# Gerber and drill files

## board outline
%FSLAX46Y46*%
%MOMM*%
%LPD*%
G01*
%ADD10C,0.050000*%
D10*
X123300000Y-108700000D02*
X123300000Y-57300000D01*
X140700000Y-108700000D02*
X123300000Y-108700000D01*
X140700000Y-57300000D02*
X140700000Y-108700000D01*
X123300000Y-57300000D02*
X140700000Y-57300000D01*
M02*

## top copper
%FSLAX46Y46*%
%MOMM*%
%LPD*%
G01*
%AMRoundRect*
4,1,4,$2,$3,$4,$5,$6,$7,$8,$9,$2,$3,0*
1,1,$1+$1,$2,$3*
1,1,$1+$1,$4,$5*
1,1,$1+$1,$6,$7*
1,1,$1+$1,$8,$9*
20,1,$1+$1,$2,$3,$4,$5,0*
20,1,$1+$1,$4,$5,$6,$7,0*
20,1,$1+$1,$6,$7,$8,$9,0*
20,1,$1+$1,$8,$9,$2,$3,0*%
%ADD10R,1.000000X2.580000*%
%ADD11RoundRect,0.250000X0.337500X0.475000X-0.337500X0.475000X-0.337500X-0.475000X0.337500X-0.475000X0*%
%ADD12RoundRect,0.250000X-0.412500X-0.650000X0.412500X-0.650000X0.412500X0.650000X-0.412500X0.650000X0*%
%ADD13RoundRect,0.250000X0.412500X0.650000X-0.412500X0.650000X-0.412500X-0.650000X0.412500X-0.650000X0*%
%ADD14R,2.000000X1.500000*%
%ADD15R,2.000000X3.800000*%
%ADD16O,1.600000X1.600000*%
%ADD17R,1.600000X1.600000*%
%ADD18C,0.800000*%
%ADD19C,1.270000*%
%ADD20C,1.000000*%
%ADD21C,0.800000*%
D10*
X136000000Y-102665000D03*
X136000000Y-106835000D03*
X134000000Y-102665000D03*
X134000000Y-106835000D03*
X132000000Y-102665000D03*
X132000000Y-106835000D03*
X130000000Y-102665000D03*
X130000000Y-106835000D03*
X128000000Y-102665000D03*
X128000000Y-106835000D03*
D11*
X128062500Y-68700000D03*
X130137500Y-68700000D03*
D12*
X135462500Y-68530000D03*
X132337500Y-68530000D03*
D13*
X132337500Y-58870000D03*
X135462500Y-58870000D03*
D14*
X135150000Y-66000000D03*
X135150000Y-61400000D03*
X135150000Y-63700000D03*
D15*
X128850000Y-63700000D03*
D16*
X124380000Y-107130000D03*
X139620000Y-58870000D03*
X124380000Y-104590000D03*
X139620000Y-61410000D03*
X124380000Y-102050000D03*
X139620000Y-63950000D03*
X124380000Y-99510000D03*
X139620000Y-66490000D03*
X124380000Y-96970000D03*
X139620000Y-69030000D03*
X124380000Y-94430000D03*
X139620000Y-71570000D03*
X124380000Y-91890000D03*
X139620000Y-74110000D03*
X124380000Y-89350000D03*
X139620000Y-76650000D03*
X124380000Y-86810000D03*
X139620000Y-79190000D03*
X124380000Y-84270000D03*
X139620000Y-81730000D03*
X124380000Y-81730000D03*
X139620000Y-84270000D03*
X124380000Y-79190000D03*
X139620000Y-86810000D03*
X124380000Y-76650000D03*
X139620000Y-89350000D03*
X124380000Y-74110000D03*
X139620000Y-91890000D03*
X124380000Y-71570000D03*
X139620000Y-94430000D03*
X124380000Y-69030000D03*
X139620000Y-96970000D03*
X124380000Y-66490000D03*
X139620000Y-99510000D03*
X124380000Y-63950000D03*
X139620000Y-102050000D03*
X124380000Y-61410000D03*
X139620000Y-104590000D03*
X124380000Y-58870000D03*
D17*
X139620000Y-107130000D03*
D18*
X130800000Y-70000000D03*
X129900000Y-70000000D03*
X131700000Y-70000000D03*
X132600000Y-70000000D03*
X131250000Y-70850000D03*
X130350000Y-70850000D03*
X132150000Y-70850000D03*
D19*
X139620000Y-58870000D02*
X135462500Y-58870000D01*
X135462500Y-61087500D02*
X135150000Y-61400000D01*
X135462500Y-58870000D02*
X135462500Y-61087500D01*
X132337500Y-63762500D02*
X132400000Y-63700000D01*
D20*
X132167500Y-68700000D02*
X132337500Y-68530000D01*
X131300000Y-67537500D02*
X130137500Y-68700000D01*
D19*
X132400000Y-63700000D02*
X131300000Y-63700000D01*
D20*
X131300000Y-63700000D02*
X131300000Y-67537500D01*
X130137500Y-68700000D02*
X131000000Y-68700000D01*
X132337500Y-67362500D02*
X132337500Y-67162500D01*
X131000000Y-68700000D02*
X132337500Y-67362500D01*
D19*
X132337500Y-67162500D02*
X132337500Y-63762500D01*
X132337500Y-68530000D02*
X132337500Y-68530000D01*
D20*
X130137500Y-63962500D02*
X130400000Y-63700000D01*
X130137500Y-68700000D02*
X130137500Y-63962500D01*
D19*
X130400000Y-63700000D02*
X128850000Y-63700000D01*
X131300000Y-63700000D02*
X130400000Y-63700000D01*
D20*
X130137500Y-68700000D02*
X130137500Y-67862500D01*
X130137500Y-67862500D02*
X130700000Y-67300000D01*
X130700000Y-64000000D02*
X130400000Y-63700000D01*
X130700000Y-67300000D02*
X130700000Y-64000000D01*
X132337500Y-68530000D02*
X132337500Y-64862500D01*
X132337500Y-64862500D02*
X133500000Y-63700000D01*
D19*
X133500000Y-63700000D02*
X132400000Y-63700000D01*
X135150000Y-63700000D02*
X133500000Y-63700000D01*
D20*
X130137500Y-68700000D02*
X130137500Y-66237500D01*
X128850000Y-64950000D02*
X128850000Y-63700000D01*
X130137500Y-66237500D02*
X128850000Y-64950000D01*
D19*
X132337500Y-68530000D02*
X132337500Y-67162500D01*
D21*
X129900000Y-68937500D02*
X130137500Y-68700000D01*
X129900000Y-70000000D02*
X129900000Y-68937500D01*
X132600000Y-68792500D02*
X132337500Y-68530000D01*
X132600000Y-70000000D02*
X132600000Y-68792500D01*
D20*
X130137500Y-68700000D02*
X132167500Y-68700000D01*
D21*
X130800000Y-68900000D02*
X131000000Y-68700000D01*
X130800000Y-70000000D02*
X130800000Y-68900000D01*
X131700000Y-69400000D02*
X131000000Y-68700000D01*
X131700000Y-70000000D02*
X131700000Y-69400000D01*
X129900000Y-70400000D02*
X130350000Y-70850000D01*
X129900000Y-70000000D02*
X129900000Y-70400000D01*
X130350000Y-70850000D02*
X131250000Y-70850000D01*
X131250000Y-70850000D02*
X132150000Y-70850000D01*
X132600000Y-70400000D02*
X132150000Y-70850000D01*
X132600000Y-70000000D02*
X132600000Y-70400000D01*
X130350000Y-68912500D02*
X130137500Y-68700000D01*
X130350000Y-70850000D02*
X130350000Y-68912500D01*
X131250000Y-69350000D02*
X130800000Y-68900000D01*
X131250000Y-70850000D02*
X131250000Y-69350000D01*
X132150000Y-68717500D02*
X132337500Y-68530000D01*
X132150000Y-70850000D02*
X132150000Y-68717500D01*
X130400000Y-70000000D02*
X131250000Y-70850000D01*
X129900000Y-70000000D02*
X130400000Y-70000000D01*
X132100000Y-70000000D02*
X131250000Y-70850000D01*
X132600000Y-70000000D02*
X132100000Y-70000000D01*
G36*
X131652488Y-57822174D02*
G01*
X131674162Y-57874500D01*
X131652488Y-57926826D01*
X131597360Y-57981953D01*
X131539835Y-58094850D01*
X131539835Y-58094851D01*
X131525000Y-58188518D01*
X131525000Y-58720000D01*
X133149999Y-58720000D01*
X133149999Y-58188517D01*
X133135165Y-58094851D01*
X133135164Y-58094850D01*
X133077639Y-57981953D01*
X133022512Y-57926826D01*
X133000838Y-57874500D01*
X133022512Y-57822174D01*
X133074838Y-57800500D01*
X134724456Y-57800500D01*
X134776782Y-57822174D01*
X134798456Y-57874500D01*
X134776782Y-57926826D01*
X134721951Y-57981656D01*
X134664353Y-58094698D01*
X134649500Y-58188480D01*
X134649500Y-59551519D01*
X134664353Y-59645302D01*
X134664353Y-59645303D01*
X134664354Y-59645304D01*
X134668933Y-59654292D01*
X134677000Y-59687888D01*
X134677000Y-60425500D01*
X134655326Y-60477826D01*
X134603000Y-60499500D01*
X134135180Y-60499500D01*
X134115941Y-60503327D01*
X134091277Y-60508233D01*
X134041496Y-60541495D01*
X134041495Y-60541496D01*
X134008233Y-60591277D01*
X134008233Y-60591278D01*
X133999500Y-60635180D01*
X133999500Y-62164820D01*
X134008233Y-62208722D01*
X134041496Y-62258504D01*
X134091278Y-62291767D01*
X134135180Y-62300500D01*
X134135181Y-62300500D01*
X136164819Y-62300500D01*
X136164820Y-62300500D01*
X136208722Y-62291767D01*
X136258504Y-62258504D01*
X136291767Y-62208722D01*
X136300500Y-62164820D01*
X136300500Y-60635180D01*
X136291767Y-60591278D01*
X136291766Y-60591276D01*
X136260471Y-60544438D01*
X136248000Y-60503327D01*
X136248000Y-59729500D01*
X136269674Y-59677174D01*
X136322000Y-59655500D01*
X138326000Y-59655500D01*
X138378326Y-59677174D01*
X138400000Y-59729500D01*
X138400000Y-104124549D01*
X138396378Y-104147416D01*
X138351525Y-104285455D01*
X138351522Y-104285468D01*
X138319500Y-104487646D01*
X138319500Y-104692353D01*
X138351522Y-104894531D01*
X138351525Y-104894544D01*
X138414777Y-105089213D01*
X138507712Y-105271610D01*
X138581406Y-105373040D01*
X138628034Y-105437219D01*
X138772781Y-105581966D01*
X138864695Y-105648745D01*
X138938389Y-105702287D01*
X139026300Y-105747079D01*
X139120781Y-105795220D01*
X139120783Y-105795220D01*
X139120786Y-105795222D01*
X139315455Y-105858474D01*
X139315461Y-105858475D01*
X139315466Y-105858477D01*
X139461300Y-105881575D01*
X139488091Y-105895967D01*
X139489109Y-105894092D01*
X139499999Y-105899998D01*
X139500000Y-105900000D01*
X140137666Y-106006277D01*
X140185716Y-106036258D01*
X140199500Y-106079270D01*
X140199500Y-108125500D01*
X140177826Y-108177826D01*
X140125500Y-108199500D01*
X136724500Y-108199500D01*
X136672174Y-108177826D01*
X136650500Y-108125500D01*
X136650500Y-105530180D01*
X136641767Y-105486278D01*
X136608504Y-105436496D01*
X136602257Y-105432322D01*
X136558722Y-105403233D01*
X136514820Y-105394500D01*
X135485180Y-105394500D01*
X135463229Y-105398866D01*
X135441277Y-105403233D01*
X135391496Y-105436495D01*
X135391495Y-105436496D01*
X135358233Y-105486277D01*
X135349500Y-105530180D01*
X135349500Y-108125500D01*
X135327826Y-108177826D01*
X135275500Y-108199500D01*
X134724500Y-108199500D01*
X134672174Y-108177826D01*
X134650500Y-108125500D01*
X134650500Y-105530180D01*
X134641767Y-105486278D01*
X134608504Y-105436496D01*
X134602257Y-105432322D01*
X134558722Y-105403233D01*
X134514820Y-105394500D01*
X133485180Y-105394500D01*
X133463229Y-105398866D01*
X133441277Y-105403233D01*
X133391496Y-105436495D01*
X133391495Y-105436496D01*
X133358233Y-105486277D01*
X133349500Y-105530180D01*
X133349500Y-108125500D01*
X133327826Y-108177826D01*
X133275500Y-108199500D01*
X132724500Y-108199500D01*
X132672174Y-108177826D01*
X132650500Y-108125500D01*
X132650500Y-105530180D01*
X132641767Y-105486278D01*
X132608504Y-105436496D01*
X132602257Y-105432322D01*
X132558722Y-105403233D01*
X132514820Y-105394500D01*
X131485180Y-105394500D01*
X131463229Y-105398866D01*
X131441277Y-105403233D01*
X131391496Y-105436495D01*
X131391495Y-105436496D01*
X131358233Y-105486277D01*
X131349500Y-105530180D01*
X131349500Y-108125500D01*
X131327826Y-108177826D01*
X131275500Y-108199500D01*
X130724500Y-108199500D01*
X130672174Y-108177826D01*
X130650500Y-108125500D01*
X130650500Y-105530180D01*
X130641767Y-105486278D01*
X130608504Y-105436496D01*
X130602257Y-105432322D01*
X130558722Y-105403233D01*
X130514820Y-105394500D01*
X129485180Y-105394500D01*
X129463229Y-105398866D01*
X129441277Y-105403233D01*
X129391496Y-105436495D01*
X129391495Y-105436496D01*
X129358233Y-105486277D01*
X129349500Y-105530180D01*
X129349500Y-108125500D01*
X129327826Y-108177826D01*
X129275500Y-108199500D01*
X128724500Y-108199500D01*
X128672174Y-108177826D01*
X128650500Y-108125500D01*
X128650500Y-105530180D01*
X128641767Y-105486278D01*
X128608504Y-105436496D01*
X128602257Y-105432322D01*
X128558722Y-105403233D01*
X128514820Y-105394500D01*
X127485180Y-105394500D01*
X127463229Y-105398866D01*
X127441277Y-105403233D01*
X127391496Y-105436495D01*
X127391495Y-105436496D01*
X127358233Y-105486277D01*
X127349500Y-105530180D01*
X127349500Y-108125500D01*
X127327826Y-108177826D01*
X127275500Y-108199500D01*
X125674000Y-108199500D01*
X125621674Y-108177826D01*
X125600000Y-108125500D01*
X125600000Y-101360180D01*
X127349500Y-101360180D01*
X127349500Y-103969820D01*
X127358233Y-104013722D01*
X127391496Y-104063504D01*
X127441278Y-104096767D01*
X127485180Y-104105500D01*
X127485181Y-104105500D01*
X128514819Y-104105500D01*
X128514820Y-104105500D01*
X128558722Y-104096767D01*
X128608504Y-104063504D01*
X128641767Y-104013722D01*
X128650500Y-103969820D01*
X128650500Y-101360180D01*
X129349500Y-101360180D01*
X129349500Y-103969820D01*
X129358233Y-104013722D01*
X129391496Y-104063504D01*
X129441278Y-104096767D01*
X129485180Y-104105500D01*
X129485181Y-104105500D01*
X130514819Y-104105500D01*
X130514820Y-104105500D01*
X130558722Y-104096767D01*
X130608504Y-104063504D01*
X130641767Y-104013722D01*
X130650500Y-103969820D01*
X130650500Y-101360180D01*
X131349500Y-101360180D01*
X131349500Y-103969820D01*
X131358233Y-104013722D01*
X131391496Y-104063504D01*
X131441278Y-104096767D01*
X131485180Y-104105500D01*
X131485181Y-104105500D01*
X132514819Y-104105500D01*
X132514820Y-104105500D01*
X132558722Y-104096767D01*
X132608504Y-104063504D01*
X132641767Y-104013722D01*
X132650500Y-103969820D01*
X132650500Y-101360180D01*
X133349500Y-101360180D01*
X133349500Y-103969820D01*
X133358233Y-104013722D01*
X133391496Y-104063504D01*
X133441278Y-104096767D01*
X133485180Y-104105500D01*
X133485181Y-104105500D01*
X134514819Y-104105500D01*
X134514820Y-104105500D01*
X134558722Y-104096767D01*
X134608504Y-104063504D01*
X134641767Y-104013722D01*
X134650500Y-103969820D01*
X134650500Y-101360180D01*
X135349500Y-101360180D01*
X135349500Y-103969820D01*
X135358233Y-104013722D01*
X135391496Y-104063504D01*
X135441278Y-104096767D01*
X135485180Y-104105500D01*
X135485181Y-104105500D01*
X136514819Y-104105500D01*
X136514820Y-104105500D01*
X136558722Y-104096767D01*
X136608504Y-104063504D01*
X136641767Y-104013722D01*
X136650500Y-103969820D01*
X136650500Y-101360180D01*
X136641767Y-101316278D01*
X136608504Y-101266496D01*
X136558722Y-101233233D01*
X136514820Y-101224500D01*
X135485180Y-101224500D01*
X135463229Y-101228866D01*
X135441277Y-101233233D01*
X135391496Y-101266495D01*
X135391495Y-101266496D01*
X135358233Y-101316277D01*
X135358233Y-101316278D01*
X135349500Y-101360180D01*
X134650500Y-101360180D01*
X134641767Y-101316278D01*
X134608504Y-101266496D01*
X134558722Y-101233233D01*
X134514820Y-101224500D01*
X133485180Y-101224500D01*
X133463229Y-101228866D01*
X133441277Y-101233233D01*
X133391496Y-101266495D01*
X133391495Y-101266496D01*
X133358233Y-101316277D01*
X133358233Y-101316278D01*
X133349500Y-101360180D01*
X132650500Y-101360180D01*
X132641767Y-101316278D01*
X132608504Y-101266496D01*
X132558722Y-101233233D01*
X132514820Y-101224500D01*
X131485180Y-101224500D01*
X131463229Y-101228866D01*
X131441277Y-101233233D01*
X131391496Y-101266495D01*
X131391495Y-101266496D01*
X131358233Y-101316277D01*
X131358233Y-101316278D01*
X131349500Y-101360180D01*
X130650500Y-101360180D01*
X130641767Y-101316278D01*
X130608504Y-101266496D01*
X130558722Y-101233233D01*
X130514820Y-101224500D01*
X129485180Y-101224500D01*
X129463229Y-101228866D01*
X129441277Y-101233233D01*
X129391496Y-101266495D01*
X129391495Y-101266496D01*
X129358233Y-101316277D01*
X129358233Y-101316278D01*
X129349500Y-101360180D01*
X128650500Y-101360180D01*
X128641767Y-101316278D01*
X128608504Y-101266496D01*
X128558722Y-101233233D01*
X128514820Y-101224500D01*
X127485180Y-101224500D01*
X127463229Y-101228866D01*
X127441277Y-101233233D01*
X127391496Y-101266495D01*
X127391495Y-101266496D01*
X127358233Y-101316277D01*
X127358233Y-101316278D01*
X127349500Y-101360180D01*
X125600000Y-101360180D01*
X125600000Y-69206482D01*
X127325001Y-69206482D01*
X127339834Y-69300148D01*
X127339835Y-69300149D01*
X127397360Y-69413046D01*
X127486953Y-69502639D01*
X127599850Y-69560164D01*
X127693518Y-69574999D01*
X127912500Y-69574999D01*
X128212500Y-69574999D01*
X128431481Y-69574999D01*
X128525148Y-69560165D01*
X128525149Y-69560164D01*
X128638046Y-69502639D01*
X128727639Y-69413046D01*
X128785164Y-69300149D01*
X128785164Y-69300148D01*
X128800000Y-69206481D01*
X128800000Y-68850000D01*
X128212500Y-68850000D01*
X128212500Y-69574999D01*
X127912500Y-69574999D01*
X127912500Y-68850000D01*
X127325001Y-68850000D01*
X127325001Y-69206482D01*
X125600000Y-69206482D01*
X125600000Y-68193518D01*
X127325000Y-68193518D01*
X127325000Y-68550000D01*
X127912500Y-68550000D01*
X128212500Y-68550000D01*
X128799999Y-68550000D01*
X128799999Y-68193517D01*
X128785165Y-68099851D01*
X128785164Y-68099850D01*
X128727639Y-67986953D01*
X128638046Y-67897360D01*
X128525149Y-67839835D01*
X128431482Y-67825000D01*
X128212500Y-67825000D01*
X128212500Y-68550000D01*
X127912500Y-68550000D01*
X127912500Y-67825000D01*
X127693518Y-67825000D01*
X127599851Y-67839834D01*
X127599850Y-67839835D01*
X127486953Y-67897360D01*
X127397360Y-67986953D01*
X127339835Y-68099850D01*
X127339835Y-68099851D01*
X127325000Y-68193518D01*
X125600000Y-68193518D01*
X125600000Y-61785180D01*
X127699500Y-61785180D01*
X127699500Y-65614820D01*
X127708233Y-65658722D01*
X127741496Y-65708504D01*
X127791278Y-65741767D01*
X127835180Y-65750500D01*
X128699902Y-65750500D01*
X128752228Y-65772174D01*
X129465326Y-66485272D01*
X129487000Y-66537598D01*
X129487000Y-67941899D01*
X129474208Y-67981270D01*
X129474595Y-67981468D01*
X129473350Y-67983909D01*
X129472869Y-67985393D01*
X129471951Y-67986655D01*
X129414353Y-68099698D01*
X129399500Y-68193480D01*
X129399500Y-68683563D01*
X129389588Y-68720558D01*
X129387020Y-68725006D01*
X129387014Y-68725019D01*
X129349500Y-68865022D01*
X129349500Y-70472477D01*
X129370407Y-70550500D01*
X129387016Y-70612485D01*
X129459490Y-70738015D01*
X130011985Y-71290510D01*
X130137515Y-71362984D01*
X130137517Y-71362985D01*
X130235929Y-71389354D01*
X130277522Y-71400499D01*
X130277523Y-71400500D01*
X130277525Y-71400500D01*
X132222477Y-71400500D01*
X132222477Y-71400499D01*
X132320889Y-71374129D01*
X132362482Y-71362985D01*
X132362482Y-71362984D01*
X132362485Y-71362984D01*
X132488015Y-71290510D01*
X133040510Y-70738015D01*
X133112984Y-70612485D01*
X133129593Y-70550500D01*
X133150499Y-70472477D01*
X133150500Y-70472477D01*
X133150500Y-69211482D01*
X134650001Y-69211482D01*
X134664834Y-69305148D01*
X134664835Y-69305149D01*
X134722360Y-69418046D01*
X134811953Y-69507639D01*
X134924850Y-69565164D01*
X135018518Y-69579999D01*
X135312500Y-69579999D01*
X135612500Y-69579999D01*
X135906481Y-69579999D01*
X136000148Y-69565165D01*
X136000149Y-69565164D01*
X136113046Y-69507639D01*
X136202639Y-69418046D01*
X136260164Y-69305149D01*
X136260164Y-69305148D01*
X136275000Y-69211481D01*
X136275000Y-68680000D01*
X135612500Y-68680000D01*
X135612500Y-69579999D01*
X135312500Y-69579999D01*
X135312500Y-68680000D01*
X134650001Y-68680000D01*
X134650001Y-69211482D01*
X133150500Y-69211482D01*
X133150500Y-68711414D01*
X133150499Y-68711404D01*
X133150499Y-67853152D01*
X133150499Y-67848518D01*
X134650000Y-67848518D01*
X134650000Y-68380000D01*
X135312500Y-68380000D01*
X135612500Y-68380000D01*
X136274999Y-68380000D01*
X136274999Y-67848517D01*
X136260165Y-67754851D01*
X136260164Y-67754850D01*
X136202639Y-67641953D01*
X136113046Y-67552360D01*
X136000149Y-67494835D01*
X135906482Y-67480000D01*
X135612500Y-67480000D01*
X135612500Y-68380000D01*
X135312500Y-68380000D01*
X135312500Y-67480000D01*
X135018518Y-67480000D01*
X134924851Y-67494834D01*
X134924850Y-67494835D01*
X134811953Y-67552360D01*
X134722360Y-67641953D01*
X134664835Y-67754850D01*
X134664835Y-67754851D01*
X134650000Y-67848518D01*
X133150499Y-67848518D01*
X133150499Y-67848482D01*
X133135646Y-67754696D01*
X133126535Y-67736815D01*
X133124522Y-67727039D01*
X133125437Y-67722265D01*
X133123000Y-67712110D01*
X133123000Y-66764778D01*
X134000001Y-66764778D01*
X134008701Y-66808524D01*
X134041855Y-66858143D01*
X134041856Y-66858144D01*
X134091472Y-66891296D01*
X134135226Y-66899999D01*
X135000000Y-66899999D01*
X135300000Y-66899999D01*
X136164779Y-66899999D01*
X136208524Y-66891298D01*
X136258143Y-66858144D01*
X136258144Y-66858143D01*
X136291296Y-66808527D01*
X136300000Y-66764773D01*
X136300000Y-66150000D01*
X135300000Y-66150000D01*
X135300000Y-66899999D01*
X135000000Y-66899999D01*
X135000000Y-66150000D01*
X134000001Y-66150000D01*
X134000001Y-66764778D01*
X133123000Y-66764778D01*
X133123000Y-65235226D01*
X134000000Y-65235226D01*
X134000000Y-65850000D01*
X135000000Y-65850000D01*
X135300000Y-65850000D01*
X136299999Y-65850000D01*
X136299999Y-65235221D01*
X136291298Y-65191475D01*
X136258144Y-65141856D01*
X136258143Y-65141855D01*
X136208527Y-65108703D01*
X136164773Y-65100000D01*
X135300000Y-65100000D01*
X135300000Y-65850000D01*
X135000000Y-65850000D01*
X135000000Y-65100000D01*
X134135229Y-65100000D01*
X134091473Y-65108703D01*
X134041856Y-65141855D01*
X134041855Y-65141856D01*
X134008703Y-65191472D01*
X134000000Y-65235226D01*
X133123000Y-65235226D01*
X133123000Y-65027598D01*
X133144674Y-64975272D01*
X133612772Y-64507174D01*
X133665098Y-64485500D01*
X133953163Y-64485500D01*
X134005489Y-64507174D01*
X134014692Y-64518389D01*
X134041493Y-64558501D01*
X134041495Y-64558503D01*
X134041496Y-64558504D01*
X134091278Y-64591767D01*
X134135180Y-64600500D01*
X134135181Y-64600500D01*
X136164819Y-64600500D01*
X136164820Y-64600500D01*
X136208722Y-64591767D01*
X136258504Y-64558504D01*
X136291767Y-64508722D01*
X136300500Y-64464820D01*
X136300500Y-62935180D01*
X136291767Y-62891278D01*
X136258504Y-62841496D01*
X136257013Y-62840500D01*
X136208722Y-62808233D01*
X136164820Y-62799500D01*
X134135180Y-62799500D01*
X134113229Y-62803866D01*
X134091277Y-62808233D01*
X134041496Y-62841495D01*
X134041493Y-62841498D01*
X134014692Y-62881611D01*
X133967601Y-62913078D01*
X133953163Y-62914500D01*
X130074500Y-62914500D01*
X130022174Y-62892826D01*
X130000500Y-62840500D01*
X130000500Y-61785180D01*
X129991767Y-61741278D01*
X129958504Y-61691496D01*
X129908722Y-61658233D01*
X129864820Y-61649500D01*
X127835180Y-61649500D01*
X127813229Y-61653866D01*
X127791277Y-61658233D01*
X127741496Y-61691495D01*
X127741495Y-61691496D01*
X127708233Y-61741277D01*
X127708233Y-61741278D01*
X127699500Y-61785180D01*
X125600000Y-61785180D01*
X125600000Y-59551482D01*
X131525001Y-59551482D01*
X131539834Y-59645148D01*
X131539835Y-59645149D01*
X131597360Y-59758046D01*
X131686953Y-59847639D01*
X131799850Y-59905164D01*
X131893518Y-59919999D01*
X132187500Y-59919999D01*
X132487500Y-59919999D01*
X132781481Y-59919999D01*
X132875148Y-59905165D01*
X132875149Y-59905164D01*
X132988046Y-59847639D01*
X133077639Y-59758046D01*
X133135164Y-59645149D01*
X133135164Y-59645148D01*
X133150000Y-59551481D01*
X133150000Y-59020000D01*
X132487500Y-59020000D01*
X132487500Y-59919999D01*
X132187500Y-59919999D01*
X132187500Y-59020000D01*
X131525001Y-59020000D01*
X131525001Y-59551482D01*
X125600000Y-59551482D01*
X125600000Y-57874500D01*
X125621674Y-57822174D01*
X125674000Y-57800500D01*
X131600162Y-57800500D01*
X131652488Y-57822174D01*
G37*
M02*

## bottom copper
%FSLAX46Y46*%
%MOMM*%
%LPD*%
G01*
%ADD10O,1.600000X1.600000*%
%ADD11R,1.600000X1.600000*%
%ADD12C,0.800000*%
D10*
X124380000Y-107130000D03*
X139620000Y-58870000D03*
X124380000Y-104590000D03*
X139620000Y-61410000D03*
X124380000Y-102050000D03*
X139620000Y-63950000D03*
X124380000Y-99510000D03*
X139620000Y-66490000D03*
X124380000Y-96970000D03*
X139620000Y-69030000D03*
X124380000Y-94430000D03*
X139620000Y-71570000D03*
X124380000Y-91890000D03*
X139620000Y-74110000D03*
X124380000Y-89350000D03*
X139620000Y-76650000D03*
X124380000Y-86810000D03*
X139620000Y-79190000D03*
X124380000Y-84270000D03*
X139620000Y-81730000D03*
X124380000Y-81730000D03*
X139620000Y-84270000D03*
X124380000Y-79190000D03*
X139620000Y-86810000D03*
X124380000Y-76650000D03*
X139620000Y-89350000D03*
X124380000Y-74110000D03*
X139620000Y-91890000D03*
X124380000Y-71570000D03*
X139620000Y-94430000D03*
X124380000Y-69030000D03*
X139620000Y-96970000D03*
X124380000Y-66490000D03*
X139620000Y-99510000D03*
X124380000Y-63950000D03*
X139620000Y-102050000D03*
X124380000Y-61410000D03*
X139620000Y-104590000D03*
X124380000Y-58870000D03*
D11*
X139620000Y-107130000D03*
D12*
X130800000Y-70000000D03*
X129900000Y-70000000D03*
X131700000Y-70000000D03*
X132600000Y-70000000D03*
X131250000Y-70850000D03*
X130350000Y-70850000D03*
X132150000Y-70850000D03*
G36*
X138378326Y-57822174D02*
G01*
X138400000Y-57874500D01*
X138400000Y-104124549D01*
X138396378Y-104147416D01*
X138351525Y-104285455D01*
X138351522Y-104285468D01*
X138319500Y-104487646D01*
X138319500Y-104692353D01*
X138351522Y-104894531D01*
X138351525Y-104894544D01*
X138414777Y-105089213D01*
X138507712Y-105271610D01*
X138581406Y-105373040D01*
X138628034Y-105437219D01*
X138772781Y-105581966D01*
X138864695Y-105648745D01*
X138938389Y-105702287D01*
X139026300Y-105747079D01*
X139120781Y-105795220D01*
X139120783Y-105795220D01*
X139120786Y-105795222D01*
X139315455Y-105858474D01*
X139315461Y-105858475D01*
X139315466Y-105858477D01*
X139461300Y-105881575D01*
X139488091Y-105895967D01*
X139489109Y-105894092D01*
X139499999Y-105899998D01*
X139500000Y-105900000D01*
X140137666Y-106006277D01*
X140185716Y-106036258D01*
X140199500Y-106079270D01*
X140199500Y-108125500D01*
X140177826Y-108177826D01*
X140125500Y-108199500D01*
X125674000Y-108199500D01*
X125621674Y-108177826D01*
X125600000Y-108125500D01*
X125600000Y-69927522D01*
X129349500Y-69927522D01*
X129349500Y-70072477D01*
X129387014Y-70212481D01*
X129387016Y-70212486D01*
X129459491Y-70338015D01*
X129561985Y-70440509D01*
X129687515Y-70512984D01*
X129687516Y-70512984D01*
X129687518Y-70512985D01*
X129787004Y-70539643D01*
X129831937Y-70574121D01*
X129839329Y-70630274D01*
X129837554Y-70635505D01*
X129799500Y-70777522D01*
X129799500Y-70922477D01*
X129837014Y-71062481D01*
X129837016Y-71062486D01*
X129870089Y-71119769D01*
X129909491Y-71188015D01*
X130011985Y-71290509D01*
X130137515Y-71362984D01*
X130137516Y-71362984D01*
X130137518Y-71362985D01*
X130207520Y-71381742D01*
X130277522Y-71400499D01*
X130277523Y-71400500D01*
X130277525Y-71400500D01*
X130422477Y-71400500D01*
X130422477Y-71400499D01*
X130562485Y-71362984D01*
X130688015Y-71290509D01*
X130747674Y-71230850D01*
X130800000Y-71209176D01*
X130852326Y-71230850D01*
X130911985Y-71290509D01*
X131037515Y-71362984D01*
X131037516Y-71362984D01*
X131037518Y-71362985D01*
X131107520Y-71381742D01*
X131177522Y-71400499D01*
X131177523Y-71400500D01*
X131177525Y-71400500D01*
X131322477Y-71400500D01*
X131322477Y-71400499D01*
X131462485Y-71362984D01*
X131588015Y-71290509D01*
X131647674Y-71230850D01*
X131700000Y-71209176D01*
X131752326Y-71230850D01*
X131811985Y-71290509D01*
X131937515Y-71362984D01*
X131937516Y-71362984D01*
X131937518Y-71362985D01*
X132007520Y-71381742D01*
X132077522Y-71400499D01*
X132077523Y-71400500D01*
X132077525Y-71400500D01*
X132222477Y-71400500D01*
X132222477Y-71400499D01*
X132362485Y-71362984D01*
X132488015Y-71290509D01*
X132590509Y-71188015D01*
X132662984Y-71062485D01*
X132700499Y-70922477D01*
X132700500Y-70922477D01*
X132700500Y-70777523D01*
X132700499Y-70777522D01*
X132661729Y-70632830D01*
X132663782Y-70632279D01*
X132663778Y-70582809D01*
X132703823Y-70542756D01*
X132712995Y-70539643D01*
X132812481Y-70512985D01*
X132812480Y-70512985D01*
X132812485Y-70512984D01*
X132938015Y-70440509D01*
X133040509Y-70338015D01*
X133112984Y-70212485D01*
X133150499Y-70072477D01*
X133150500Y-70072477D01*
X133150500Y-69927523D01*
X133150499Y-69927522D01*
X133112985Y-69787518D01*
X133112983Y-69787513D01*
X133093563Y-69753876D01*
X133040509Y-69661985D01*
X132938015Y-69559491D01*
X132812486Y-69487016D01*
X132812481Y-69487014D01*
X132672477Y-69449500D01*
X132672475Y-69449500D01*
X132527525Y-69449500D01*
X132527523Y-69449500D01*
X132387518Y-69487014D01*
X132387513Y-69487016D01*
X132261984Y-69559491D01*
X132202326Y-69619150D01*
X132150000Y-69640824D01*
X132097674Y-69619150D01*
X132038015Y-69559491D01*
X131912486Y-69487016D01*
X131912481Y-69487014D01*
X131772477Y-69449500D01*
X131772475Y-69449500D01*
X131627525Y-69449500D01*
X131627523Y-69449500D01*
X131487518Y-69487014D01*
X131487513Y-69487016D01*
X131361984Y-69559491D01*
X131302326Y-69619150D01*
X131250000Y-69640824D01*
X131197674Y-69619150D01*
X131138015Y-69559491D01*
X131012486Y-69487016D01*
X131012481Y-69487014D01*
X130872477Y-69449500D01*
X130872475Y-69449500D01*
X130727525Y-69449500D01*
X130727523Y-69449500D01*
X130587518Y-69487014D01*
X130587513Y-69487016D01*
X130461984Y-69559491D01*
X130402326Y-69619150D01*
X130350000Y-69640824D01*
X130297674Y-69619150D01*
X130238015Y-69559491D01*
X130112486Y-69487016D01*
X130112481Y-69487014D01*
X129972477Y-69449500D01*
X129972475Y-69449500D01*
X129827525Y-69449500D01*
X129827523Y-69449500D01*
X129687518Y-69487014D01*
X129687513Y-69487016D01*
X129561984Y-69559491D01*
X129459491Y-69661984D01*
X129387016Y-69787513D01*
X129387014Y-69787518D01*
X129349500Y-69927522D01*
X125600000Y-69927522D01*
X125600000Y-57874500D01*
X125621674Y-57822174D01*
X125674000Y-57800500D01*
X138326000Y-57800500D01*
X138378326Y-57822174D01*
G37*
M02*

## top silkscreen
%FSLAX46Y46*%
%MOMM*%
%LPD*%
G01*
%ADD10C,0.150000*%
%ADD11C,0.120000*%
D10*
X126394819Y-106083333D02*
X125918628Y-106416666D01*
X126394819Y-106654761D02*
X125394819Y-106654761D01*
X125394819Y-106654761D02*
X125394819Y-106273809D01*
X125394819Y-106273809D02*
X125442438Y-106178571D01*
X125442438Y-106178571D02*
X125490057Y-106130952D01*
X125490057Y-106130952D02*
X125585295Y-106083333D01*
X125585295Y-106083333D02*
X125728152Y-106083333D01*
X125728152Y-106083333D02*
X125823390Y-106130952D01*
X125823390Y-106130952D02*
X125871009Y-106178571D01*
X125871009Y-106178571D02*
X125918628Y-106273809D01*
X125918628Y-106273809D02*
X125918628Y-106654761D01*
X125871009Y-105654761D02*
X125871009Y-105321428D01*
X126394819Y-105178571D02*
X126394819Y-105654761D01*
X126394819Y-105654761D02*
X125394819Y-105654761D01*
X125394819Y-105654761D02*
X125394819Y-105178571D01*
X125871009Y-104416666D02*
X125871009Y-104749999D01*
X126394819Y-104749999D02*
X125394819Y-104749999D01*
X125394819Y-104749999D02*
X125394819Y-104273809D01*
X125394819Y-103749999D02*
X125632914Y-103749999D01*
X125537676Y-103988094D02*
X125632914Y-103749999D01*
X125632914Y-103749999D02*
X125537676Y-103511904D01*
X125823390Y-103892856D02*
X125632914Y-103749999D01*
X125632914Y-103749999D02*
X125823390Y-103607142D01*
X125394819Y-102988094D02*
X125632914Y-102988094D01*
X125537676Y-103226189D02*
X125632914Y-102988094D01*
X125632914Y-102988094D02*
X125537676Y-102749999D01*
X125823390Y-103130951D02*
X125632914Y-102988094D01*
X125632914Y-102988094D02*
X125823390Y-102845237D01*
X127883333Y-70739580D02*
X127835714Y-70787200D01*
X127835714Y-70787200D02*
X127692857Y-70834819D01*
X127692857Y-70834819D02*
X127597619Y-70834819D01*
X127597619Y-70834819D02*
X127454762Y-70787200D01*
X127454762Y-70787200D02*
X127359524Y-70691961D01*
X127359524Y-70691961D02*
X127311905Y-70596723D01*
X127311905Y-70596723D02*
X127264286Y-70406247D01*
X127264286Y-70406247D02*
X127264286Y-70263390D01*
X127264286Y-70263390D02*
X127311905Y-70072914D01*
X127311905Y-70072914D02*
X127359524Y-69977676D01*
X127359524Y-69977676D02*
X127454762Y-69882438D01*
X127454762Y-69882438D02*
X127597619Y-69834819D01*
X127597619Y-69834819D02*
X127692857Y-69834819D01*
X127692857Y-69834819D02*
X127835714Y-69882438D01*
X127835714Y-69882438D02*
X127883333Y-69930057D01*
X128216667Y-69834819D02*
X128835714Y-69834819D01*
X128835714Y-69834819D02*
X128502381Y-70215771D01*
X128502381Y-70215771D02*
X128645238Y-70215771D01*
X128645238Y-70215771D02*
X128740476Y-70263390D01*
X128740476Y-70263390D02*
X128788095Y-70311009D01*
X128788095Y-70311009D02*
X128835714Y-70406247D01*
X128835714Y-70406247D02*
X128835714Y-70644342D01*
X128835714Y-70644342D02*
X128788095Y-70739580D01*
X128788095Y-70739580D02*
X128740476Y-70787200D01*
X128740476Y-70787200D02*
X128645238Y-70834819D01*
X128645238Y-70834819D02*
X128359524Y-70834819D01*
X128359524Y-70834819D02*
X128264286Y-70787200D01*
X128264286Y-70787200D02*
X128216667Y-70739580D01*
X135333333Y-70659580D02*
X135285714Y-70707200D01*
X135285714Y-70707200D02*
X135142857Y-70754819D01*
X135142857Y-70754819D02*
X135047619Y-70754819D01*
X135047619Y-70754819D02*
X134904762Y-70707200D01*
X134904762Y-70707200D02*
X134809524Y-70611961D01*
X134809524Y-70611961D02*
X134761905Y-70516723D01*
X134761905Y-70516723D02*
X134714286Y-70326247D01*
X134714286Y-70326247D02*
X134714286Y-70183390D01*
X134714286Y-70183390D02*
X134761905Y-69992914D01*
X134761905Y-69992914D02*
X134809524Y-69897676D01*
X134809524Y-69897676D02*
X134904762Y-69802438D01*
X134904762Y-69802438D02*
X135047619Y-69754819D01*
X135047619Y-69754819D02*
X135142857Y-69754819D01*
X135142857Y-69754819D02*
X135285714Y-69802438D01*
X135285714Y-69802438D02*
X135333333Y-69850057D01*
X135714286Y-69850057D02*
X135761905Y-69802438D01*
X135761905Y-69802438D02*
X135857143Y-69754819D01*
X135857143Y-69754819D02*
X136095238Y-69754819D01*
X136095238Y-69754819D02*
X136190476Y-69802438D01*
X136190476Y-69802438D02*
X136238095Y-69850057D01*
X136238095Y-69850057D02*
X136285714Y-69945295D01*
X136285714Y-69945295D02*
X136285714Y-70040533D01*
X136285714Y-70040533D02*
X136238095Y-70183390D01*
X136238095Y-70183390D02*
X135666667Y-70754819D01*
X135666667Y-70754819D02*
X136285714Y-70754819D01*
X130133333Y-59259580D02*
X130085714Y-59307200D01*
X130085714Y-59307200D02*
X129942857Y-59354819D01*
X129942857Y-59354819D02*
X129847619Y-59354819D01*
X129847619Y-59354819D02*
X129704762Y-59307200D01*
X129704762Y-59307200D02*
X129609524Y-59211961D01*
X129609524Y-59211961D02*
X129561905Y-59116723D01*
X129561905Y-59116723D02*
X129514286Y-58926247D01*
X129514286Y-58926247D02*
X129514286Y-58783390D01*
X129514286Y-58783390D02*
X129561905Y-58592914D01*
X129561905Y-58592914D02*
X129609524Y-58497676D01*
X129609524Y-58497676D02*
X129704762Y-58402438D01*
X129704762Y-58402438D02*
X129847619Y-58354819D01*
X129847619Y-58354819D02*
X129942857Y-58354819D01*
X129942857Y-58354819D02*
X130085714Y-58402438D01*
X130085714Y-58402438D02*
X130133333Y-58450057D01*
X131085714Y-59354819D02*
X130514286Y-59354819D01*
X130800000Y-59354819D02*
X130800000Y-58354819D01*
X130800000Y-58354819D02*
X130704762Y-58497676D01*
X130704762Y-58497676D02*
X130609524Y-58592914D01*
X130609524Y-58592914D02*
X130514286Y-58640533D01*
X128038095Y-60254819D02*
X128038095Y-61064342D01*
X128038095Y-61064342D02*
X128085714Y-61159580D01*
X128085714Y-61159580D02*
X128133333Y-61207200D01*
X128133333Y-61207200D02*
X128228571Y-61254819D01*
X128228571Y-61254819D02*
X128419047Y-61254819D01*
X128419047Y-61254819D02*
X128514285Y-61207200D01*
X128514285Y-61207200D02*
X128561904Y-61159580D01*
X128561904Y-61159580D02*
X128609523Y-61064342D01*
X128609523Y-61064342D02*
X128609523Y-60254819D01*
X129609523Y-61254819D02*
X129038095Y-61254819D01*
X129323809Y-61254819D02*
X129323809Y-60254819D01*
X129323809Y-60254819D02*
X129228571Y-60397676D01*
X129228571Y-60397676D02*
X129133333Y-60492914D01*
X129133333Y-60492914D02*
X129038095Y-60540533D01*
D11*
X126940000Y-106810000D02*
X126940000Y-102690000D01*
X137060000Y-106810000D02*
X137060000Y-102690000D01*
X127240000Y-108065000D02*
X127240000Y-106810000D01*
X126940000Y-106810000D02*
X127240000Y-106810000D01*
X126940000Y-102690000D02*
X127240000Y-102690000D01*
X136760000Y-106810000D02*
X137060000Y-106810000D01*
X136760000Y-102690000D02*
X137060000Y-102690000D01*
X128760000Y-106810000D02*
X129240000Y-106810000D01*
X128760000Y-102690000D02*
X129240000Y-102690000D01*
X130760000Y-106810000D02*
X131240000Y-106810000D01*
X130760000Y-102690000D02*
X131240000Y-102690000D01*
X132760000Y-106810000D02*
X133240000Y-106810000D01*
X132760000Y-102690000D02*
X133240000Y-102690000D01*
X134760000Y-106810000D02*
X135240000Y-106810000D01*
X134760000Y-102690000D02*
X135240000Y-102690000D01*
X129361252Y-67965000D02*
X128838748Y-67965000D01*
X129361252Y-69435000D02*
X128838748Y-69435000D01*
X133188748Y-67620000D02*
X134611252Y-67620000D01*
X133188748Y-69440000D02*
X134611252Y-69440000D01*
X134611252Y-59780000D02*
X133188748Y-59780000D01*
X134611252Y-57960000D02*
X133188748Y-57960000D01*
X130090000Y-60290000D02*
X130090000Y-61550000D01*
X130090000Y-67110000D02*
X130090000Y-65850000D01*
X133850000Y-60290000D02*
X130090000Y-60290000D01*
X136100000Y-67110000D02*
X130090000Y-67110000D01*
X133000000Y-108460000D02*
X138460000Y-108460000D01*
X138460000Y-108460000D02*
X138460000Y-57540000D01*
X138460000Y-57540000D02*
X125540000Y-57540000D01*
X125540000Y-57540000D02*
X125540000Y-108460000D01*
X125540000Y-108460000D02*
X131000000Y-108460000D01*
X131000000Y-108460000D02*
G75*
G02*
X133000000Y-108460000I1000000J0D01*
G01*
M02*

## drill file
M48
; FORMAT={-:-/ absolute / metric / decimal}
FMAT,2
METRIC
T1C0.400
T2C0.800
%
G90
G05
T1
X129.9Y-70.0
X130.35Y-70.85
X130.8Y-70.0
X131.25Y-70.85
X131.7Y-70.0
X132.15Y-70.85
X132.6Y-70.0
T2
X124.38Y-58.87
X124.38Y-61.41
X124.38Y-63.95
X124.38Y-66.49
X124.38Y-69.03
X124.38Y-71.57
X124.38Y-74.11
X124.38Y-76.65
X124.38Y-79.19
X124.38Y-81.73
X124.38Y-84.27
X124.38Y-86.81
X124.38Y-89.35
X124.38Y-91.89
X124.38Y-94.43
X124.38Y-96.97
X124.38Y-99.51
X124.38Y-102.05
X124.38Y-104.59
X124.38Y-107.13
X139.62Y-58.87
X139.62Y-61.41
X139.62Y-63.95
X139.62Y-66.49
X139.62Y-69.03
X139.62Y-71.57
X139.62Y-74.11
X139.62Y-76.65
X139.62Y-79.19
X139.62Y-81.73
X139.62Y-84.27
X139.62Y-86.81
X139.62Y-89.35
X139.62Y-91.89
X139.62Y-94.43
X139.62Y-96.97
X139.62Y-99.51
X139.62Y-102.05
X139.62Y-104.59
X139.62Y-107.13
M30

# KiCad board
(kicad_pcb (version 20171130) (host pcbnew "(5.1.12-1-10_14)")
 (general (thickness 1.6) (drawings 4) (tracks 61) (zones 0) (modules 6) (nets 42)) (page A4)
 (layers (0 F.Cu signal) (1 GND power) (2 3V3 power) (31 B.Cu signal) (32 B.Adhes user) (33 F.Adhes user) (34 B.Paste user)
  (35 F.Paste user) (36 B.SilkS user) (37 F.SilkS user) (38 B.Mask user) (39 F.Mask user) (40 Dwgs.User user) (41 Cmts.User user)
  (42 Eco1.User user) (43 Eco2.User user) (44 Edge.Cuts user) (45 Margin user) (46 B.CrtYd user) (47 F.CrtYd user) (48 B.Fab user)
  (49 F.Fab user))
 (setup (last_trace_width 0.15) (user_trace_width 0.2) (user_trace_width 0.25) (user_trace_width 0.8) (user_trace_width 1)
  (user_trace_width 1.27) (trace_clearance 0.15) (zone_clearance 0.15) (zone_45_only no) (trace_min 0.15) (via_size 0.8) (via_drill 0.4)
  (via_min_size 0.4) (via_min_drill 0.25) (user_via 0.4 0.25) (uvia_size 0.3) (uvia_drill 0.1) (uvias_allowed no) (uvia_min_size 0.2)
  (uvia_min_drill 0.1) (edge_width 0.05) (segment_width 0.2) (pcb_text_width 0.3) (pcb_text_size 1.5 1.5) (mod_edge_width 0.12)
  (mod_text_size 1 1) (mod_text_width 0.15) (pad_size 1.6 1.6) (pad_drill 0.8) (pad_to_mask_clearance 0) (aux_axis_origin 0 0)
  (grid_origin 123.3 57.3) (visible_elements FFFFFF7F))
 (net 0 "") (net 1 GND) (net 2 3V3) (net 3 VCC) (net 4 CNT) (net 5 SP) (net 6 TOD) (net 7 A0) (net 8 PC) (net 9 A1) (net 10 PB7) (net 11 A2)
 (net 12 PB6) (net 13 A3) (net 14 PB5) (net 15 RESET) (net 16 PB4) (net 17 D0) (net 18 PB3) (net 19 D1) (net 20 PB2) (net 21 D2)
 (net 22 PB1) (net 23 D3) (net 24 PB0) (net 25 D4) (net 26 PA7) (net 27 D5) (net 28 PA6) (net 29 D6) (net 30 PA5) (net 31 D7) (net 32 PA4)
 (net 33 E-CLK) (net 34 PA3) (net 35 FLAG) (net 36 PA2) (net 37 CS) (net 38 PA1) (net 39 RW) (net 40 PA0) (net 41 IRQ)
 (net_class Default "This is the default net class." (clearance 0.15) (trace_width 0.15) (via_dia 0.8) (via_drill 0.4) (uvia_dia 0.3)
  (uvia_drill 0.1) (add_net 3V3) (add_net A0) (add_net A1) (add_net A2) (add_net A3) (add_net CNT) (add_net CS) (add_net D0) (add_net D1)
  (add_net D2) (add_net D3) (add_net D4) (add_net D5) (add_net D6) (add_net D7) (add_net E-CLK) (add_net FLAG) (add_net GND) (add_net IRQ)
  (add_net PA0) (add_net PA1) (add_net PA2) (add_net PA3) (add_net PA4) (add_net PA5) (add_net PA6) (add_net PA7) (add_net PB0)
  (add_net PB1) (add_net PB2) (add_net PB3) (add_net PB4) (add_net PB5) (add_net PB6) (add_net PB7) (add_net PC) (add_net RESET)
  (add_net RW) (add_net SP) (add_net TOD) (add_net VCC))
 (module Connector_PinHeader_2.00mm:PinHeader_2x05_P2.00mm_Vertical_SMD (layer F.Cu) (at 132 104.75 90)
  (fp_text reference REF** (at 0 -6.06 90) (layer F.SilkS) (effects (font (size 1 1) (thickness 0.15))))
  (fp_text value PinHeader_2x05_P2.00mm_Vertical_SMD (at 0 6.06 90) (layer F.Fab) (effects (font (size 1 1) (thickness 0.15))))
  (fp_line (start -2.06 -5.06) (end 2.06 -5.06) (layer F.SilkS) (width 0.12))
  (fp_line (start -2.06 5.06) (end 2.06 5.06) (layer F.SilkS) (width 0.12))
  (fp_line (start -3.315 -4.76) (end -2.06 -4.76) (layer F.SilkS) (width 0.12))
  (fp_line (start -2.06 -5.06) (end -2.06 -4.76) (layer F.SilkS) (width 0.12))
  (fp_line (start 2.06 -5.06) (end 2.06 -4.76) (layer F.SilkS) (width 0.12))
  (fp_line (start -2.06 4.76) (end -2.06 5.06) (layer F.SilkS) (width 0.12))
  (fp_line (start 2.06 4.76) (end 2.06 5.06) (layer F.SilkS) (width 0.12))
  (fp_line (start -2.06 -3.24) (end -2.06 -2.76) (layer F.SilkS) (width 0.12))
  (fp_line (start 2.06 -3.24) (end 2.06 -2.76) (layer F.SilkS) (width 0.12))
  (fp_line (start -2.06 -1.24) (end -2.06 -0.76) (layer F.SilkS) (width 0.12))
  (fp_line (start 2.06 -1.24) (end 2.06 -0.76) (layer F.SilkS) (width 0.12))
  (fp_line (start -2.06 0.76) (end -2.06 1.24) (layer F.SilkS) (width 0.12))
  (fp_line (start 2.06 0.76) (end 2.06 1.24) (layer F.SilkS) (width 0.12))
  (fp_line (start -2.06 2.76) (end -2.06 3.24) (layer F.SilkS) (width 0.12))
  (fp_line (start 2.06 2.76) (end 2.06 3.24) (layer F.SilkS) (width 0.12))
  (pad 10 smd rect (at 2.085 4 90) (size 2.58 1) (layers F.Cu F.Paste F.Mask))
  (pad 9 smd rect (at -2.085 4 90) (size 2.58 1) (layers F.Cu F.Paste F.Mask))
  (pad 8 smd rect (at 2.085 2 90) (size 2.58 1) (layers F.Cu F.Paste F.Mask))
  (pad 7 smd rect (at -2.085 2 90) (size 2.58 1) (layers F.Cu F.Paste F.Mask))
  (pad 6 smd rect (at 2.085 0 90) (size 2.58 1) (layers F.Cu F.Paste F.Mask))
  (pad 5 smd rect (at -2.085 0 90) (size 2.58 1) (layers F.Cu F.Paste F.Mask))
  (pad 4 smd rect (at 2.085 -2 90) (size 2.58 1) (layers F.Cu F.Paste F.Mask))
  (pad 3 smd rect (at -2.085 -2 90) (size 2.58 1) (layers F.Cu F.Paste F.Mask))
  (pad 2 smd rect (at 2.085 -4 90) (size 2.58 1) (layers F.Cu F.Paste F.Mask))
  (pad 1 smd rect (at -2.085 -4 90) (size 2.58 1) (layers F.Cu F.Paste F.Mask)))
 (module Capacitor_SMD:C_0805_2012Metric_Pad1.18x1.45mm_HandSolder (layer F.Cu) (at 129.1 68.7 180)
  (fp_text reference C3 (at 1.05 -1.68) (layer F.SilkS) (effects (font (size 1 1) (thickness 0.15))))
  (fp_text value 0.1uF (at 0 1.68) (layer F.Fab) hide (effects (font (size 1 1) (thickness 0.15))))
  (fp_line (start -0.261252 0.735) (end 0.261252 0.735) (layer F.SilkS) (width 0.12))
  (fp_line (start -0.261252 -0.735) (end 0.261252 -0.735) (layer F.SilkS) (width 0.12))
  (pad 2 smd roundrect (at 1.0375 0 180) (size 1.175 1.45) (layers F.Cu F.Paste F.Mask) (roundrect_rratio 0.212766) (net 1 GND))
  (pad 1 smd roundrect (at -1.0375 0 180) (size 1.175 1.45) (layers F.Cu F.Paste F.Mask) (roundrect_rratio 0.212766) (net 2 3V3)))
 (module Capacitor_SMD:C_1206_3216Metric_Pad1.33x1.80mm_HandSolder (layer F.Cu) (at 133.9 68.53)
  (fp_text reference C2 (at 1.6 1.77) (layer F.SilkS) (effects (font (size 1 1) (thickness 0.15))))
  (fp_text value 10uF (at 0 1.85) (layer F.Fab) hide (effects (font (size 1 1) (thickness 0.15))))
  (fp_line (start -0.711252 -0.91) (end 0.711252 -0.91) (layer F.SilkS) (width 0.12))
  (fp_line (start -0.711252 0.91) (end 0.711252 0.91) (layer F.SilkS) (width 0.12))
  (pad 2 smd roundrect (at 1.5625 0) (size 1.325 1.8) (layers F.Cu F.Paste F.Mask) (roundrect_rratio 0.188679) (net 1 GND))
  (pad 1 smd roundrect (at -1.5625 0) (size 1.325 1.8) (layers F.Cu F.Paste F.Mask) (roundrect_rratio 0.188679) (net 2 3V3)))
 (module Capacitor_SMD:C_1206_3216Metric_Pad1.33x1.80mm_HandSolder (layer F.Cu) (at 133.9 58.87 180)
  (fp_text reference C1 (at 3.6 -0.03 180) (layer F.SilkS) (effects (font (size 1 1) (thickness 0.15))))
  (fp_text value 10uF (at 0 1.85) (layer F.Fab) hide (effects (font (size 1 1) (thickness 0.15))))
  (fp_line (start -0.711252 -0.91) (end 0.711252 -0.91) (layer F.SilkS) (width 0.12))
  (fp_line (start -0.711252 0.91) (end 0.711252 0.91) (layer F.SilkS) (width 0.12))
  (pad 2 smd roundrect (at 1.5625 0 180) (size 1.325 1.8) (layers F.Cu F.Paste F.Mask) (roundrect_rratio 0.188679) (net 1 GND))
  (pad 1 smd roundrect (at -1.5625 0 180) (size 1.325 1.8) (layers F.Cu F.Paste F.Mask) (roundrect_rratio 0.188679) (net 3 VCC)))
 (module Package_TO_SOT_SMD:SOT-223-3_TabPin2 (layer F.Cu) (at 132 63.7 180)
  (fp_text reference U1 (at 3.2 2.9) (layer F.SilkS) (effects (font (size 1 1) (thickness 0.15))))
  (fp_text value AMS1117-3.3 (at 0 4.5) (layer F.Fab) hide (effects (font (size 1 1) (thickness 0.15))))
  (fp_line (start 1.91 3.41) (end 1.91 2.15) (layer F.SilkS) (width 0.12))
  (fp_line (start 1.91 -3.41) (end 1.91 -2.15) (layer F.SilkS) (width 0.12))
  (fp_line (start -1.85 3.41) (end 1.91 3.41) (layer F.SilkS) (width 0.12))
  (fp_line (start -4.1 -3.41) (end 1.91 -3.41) (layer F.SilkS) (width 0.12))
  (pad 1 smd rect (at -3.15 -2.3 180) (size 2 1.5) (layers F.Cu F.Paste F.Mask) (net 1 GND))
  (pad 3 smd rect (at -3.15 2.3 180) (size 2 1.5) (layers F.Cu F.Paste F.Mask) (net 3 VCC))
  (pad 2 smd rect (at -3.15 0 180) (size 2 1.5) (layers F.Cu F.Paste F.Mask) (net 2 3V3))
  (pad 2 smd rect (at 3.15 0 180) (size 2 3.8) (layers F.Cu F.Paste F.Mask) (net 2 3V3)))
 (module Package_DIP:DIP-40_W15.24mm (layer F.Cu) (at 132 83 180)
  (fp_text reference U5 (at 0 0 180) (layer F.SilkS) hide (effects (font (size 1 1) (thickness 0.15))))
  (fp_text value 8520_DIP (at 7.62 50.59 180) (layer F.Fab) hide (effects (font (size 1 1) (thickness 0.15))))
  (fp_line (start -1 -25.46) (end -6.46 -25.46) (layer F.SilkS) (width 0.12))
  (fp_line (start -6.46 -25.46) (end -6.46 25.46) (layer F.SilkS) (width 0.12))
  (fp_line (start -6.46 25.46) (end 6.46 25.46) (layer F.SilkS) (width 0.12))
  (fp_line (start 6.46 25.46) (end 6.46 -25.46) (layer F.SilkS) (width 0.12))
  (fp_line (start 6.46 -25.46) (end 1 -25.46) (layer F.SilkS) (width 0.12))
  (fp_arc (start 0 -25.46) (end -1 -25.46) (angle -180) (layer F.SilkS) (width 0.12))
  (pad 40 thru_hole oval (at 7.62 -24.13 180) (size 1.6 1.6) (drill 0.8) (layers *.Cu *.Mask) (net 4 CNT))
  (pad 20 thru_hole oval (at -7.62 24.13 180) (size 1.6 1.6) (drill 0.8) (layers *.Cu *.Mask) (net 3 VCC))
  (pad 39 thru_hole oval (at 7.62 -21.59 180) (size 1.6 1.6) (drill 0.8) (layers *.Cu *.Mask) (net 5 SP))
  (pad 19 thru_hole oval (at -7.62 21.59 180) (size 1.6 1.6) (drill 0.8) (layers *.Cu *.Mask) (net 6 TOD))
  (pad 38 thru_hole oval (at 7.62 -19.05 180) (size 1.6 1.6) (drill 0.8) (layers *.Cu *.Mask) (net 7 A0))
  (pad 18 thru_hole oval (at -7.62 19.05 180) (size 1.6 1.6) (drill 0.8) (layers *.Cu *.Mask) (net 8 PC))
  (pad 37 thru_hole oval (at 7.62 -16.51 180) (size 1.6 1.6) (drill 0.8) (layers *.Cu *.Mask) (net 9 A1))
  (pad 17 thru_hole oval (at -7.62 16.51 180) (size 1.6 1.6) (drill 0.8) (layers *.Cu *.Mask) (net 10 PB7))
  (pad 36 thru_hole oval (at 7.62 -13.97 180) (size 1.6 1.6) (drill 0.8) (layers *.Cu *.Mask) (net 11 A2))
  (pad 16 thru_hole oval (at -7.62 13.97 180) (size 1.6 1.6) (drill 0.8) (layers *.Cu *.Mask) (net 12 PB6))
  (pad 35 thru_hole oval (at 7.62 -11.43 180) (size 1.6 1.6) (drill 0.8) (layers *.Cu *.Mask) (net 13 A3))
  (pad 15 thru_hole oval (at -7.62 11.43 180) (size 1.6 1.6) (drill 0.8) (layers *.Cu *.Mask) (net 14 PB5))
  (pad 34 thru_hole oval (at 7.62 -8.89 180) (size 1.6 1.6) (drill 0.8) (layers *.Cu *.Mask) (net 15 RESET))
  (pad 14 thru_hole oval (at -7.62 8.89 180) (size 1.6 1.6) (drill 0.8) (layers *.Cu *.Mask) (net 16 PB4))
  (pad 33 thru_hole oval (at 7.62 -6.35 180) (size 1.6 1.6) (drill 0.8) (layers *.Cu *.Mask) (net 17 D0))
  (pad 13 thru_hole oval (at -7.62 6.35 180) (size 1.6 1.6) (drill 0.8) (layers *.Cu *.Mask) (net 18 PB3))
  (pad 32 thru_hole oval (at 7.62 -3.81 180) (size 1.6 1.6) (drill 0.8) (layers *.Cu *.Mask) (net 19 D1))
  (pad 12 thru_hole oval (at -7.62 3.81 180) (size 1.6 1.6) (drill 0.8) (layers *.Cu *.Mask) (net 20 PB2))
  (pad 31 thru_hole oval (at 7.62 -1.27 180) (size 1.6 1.6) (drill 0.8) (layers *.Cu *.Mask) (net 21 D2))
  (pad 11 thru_hole oval (at -7.62 1.27 180) (size 1.6 1.6) (drill 0.8) (layers *.Cu *.Mask) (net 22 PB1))
  (pad 30 thru_hole oval (at 7.62 1.27 180) (size 1.6 1.6) (drill 0.8) (layers *.Cu *.Mask) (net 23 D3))
  (pad 10 thru_hole oval (at -7.62 -1.27 180) (size 1.6 1.6) (drill 0.8) (layers *.Cu *.Mask) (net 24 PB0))
  (pad 29 thru_hole oval (at 7.62 3.81 180) (size 1.6 1.6) (drill 0.8) (layers *.Cu *.Mask) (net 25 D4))
  (pad 9 thru_hole oval (at -7.62 -3.81 180) (size 1.6 1.6) (drill 0.8) (layers *.Cu *.Mask) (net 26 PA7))
  (pad 28 thru_hole oval (at 7.62 6.35 180) (size 1.6 1.6) (drill 0.8) (layers *.Cu *.Mask) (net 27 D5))
  (pad 8 thru_hole oval (at -7.62 -6.35 180) (size 1.6 1.6) (drill 0.8) (layers *.Cu *.Mask) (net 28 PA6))
  (pad 27 thru_hole oval (at 7.62 8.89 180) (size 1.6 1.6) (drill 0.8) (layers *.Cu *.Mask) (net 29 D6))
  (pad 7 thru_hole oval (at -7.62 -8.89 180) (size 1.6 1.6) (drill 0.8) (layers *.Cu *.Mask) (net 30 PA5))
  (pad 26 thru_hole oval (at 7.62 11.43 180) (size 1.6 1.6) (drill 0.8) (layers *.Cu *.Mask) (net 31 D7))
  (pad 6 thru_hole oval (at -7.62 -11.43 180) (size 1.6 1.6) (drill 0.8) (layers *.Cu *.Mask) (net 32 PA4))
  (pad 25 thru_hole oval (at 7.62 13.97 180) (size 1.6 1.6) (drill 0.8) (layers *.Cu *.Mask) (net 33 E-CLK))
  (pad 5 thru_hole oval (at -7.62 -13.97 180) (size 1.6 1.6) (drill 0.8) (layers *.Cu *.Mask) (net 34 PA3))
  (pad 24 thru_hole oval (at 7.62 16.51 180) (size 1.6 1.6) (drill 0.8) (layers *.Cu *.Mask) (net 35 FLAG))
  (pad 4 thru_hole oval (at -7.62 -16.51 180) (size 1.6 1.6) (drill 0.8) (layers *.Cu *.Mask) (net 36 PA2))
  (pad 23 thru_hole oval (at 7.62 19.05 180) (size 1.6 1.6) (drill 0.8) (layers *.Cu *.Mask) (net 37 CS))
  (pad 3 thru_hole oval (at -7.62 -19.05 180) (size 1.6 1.6) (drill 0.8) (layers *.Cu *.Mask) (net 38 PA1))
  (pad 22 thru_hole oval (at 7.62 21.59 180) (size 1.6 1.6) (drill 0.8) (layers *.Cu *.Mask) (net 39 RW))
  (pad 2 thru_hole oval (at -7.62 -21.59 180) (size 1.6 1.6) (drill 0.8) (layers *.Cu *.Mask) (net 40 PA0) (clearance 0.5))
  (pad 21 thru_hole oval (at 7.62 24.13 180) (size 1.6 1.6) (drill 0.8) (layers *.Cu *.Mask) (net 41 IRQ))
  (pad 1 thru_hole rect (at -7.62 -24.13 180) (size 1.6 1.6) (drill 0.8) (layers *.Cu *.Mask) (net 1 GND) (zone_connect 2)))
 (gr_line (start 123.3 108.7) (end 123.3 57.3) (layer Edge.Cuts) (width 0.05))
 (gr_line (start 140.7 108.7) (end 123.3 108.7) (layer Edge.Cuts) (width 0.05))
 (gr_line (start 140.7 57.3) (end 140.7 108.7) (layer Edge.Cuts) (width 0.05))
 (gr_line (start 123.3 57.3) (end 140.7 57.3) (layer Edge.Cuts) (width 0.05))
 (segment (start 139.62 58.87) (end 135.4625 58.87) (width 1.27) (layer F.Cu) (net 3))
 (segment (start 135.4625 61.0875) (end 135.15 61.4) (width 1.27) (layer F.Cu) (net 3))
 (segment (start 135.4625 58.87) (end 135.4625 61.0875) (width 1.27) (layer F.Cu) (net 3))
 (segment (start 132.3375 63.7625) (end 132.4 63.7) (width 1.27) (layer F.Cu) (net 2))
 (segment (start 132.1675 68.7) (end 132.3375 68.53) (width 1) (layer F.Cu) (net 2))
 (segment (start 131.3 67.5375) (end 130.1375 68.7) (width 1) (layer F.Cu) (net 2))
 (segment (start 132.4 63.7) (end 131.3 63.7) (width 1.27) (layer F.Cu) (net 2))
 (segment (start 131.3 63.7) (end 131.3 67.5375) (width 1) (layer F.Cu) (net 2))
 (segment (start 130.1375 68.7) (end 131 68.7) (width 1) (layer F.Cu) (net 2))
 (segment (start 132.3375 67.3625) (end 132.3375 67.1625) (width 1) (layer F.Cu) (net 2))
 (segment (start 131 68.7) (end 132.3375 67.3625) (width 1) (layer F.Cu) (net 2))
 (segment (start 132.3375 67.1625) (end 132.3375 63.7625) (width 1.27) (layer F.Cu) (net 2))
 (segment (start 132.3375 68.53) (end 132.3375 68.53) (width 1.27) (layer F.Cu) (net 2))
 (segment (start 130.1375 63.9625) (end 130.4 63.7) (width 1) (layer F.Cu) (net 2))
 (segment (start 130.1375 68.7) (end 130.1375 63.9625) (width 1) (layer F.Cu) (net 2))
 (segment (start 130.4 63.7) (end 128.85 63.7) (width 1.27) (layer F.Cu) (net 2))
 (segment (start 131.3 63.7) (end 130.4 63.7) (width 1.27) (layer F.Cu) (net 2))
 (segment (start 130.1375 68.7) (end 130.1375 67.8625) (width 1) (layer F.Cu) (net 2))
 (segment (start 130.1375 67.8625) (end 130.7 67.3) (width 1) (layer F.Cu) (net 2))
 (segment (start 130.7 64) (end 130.4 63.7) (width 1) (layer F.Cu) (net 2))
 (segment (start 130.7 67.3) (end 130.7 64) (width 1) (layer F.Cu) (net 2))
 (segment (start 132.3375 68.53) (end 132.3375 64.8625) (width 1) (layer F.Cu) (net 2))
 (segment (start 132.3375 64.8625) (end 133.5 63.7) (width 1) (layer F.Cu) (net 2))
 (segment (start 133.5 63.7) (end 132.4 63.7) (width 1.27) (layer F.Cu) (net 2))
 (segment (start 135.15 63.7) (end 133.5 63.7) (width 1.27) (layer F.Cu) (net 2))
 (segment (start 130.1375 68.7) (end 130.1375 66.2375) (width 1) (layer F.Cu) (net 2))
 (segment (start 128.85 64.95) (end 128.85 63.7) (width 1) (layer F.Cu) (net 2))
 (segment (start 130.1375 66.2375) (end 128.85 64.95) (width 1) (layer F.Cu) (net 2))
 (segment (start 132.3375 68.53) (end 132.3375 67.1625) (width 1.27) (layer F.Cu) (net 2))
 (via (at 130.8 70) (size 0.8) (drill 0.4) (layers F.Cu B.Cu) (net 2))
 (via (at 129.9 70) (size 0.8) (drill 0.4) (layers F.Cu B.Cu) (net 2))
 (via (at 131.7 70) (size 0.8) (drill 0.4) (layers F.Cu B.Cu) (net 2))
 (via (at 132.6 70) (size 0.8) (drill 0.4) (layers F.Cu B.Cu) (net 2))
 (via (at 131.25 70.85) (size 0.8) (drill 0.4) (layers F.Cu B.Cu) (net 2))
 (via (at 130.35 70.85) (size 0.8) (drill 0.4) (layers F.Cu B.Cu) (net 2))
 (via (at 132.15 70.85) (size 0.8) (drill 0.4) (layers F.Cu B.Cu) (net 2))
 (segment (start 129.9 68.9375) (end 130.1375 68.7) (width 0.8) (layer F.Cu) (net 2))
 (segment (start 129.9 70) (end 129.9 68.9375) (width 0.8) (layer F.Cu) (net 2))
 (segment (start 132.6 68.7925) (end 132.3375 68.53) (width 0.8) (layer F.Cu) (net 2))
 (segment (start 132.6 70) (end 132.6 68.7925) (width 0.8) (layer F.Cu) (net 2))
 (segment (start 130.1375 68.7) (end 132.1675 68.7) (width 1) (layer F.Cu) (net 2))
 (segment (start 130.8 68.9) (end 131 68.7) (width 0.8) (layer F.Cu) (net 2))
 (segment (start 130.8 70) (end 130.8 68.9) (width 0.8) (layer F.Cu) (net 2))
 (segment (start 131.7 69.4) (end 131 68.7) (width 0.8) (layer F.Cu) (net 2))
 (segment (start 131.7 70) (end 131.7 69.4) (width 0.8) (layer F.Cu) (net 2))
 (segment (start 129.9 70.4) (end 130.35 70.85) (width 0.8) (layer F.Cu) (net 2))
 (segment (start 129.9 70) (end 129.9 70.4) (width 0.8) (layer F.Cu) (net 2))
 (segment (start 130.35 70.85) (end 131.25 70.85) (width 0.8) (layer F.Cu) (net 2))
 (segment (start 131.25 70.85) (end 132.15 70.85) (width 0.8) (layer F.Cu) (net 2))
 (segment (start 132.6 70.4) (end 132.15 70.85) (width 0.8) (layer F.Cu) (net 2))
 (segment (start 132.6 70) (end 132.6 70.4) (width 0.8) (layer F.Cu) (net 2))
 (segment (start 130.35 68.9125) (end 130.1375 68.7) (width 0.8) (layer F.Cu) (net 2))
 (segment (start 130.35 70.85) (end 130.35 68.9125) (width 0.8) (layer F.Cu) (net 2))
 (segment (start 131.25 69.35) (end 130.8 68.9) (width 0.8) (layer F.Cu) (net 2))
 (segment (start 131.25 70.85) (end 131.25 69.35) (width 0.8) (layer F.Cu) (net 2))
 (segment (start 132.15 68.7175) (end 132.3375 68.53) (width 0.8) (layer F.Cu) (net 2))
 (segment (start 132.15 70.85) (end 132.15 68.7175) (width 0.8) (layer F.Cu) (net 2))
 (segment (start 130.4 70) (end 131.25 70.85) (width 0.8) (layer F.Cu) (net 2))
 (segment (start 129.9 70) (end 130.4 70) (width 0.8) (layer F.Cu) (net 2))
 (segment (start 132.1 70) (end 131.25 70.85) (width 0.8) (layer F.Cu) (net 2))
 (segment (start 132.6 70) (end 132.1 70) (width 0.8) (layer F.Cu) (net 2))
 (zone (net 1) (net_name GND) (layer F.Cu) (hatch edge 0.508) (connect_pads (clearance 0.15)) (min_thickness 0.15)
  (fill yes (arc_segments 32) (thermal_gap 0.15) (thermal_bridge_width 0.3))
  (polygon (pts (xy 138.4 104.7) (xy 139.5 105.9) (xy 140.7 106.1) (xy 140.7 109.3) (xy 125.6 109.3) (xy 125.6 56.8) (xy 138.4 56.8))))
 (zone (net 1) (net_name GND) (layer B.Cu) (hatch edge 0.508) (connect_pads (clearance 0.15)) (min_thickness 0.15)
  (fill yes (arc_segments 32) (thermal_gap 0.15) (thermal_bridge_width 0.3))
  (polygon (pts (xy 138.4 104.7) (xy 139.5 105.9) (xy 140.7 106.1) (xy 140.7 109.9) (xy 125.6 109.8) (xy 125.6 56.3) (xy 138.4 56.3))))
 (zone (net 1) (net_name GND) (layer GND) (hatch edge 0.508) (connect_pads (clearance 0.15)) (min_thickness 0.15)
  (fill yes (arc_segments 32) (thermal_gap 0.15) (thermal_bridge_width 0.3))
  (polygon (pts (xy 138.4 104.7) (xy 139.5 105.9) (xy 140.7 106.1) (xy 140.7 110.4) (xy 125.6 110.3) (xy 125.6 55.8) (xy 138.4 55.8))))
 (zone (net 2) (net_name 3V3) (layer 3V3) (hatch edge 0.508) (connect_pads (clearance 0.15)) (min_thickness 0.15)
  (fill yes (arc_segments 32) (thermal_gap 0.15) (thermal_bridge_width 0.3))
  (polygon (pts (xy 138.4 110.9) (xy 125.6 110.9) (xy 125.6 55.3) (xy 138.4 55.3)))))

